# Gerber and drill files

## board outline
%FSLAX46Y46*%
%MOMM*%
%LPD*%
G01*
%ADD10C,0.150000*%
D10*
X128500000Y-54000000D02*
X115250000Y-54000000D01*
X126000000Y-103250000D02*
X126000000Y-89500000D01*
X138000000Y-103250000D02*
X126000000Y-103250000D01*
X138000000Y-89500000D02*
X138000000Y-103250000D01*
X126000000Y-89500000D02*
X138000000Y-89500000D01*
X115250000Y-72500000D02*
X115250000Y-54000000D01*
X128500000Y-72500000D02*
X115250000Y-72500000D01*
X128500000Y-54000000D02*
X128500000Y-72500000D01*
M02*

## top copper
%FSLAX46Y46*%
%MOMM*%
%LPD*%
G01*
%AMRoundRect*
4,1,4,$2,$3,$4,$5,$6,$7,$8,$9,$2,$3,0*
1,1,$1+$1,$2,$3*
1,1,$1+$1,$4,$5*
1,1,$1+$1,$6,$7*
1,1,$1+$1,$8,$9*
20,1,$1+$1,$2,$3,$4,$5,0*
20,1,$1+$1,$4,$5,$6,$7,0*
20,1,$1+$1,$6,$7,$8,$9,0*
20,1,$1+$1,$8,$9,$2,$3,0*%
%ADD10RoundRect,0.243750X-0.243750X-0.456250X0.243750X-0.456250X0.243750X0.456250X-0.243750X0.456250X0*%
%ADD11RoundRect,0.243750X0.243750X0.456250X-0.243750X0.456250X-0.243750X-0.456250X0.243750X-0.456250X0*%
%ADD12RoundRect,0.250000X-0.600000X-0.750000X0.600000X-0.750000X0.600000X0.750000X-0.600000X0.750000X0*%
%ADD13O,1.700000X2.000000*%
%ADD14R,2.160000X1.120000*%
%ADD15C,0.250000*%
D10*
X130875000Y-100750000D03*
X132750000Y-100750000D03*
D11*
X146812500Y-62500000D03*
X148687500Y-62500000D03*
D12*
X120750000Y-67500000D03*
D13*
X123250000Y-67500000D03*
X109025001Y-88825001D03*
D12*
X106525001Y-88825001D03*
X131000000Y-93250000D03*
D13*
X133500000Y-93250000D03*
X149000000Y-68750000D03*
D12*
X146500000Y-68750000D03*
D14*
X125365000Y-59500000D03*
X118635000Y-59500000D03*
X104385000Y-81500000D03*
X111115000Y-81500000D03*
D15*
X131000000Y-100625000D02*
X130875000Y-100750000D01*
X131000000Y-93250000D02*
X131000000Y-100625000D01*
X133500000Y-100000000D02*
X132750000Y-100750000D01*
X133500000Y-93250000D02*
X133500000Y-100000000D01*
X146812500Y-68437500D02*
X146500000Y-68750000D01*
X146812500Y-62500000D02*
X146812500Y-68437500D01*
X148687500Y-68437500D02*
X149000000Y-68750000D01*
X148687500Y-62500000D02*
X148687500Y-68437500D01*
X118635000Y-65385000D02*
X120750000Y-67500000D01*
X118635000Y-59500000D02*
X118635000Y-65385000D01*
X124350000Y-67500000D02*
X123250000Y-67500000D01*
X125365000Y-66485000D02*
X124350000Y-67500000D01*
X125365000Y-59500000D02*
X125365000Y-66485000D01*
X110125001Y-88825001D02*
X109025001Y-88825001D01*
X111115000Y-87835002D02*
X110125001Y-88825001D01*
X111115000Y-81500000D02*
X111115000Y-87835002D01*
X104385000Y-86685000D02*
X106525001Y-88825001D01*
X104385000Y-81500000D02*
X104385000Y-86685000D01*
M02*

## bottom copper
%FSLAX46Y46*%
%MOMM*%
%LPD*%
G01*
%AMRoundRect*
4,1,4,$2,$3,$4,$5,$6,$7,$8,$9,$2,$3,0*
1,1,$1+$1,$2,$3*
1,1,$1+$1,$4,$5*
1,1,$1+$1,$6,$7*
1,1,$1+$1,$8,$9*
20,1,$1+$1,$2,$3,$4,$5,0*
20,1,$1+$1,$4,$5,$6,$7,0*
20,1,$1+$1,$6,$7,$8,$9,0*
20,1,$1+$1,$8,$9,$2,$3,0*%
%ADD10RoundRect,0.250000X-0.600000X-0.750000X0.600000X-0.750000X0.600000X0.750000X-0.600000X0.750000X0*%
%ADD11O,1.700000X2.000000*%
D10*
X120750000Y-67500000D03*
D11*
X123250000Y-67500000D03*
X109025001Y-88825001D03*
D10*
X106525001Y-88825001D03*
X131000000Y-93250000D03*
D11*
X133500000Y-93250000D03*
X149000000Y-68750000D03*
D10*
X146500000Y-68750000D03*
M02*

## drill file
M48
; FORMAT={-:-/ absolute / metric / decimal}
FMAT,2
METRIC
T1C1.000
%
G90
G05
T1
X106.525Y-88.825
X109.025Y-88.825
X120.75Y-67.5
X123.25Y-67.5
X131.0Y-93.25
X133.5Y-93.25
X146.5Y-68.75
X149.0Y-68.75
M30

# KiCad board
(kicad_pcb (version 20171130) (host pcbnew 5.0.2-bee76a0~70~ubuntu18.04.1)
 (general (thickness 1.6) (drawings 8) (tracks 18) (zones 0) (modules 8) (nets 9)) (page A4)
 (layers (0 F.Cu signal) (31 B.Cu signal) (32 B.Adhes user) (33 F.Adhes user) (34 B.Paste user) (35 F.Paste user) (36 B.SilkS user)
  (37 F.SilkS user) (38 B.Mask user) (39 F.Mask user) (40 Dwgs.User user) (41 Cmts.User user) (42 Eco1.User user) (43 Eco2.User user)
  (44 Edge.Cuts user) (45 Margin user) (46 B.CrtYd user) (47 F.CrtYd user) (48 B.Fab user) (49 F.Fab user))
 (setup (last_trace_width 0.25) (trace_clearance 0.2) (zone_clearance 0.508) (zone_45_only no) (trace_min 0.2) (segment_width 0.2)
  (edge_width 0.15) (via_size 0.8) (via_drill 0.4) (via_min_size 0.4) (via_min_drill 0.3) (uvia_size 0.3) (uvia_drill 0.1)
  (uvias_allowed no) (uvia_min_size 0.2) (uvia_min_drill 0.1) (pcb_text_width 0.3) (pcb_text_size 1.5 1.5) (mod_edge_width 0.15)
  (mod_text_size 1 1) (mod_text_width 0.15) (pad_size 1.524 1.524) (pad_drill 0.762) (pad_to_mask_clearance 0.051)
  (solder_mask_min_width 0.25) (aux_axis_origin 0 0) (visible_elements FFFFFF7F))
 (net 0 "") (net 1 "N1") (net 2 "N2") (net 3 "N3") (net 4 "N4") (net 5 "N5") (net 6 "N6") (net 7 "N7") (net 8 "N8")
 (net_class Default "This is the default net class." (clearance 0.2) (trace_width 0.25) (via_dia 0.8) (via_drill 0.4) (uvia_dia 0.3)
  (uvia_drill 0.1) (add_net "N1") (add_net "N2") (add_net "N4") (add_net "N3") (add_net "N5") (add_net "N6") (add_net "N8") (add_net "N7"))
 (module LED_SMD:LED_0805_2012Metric (layer F.Cu) (at 131.8125 100.75)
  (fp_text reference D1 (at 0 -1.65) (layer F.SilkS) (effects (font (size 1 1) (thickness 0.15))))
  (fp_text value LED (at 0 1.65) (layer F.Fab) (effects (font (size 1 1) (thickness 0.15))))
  (pad 1 smd roundrect (at -0.9375 0) (size 0.975 1.4) (layers F.Cu F.Paste F.Mask) (roundrect_rratio 0.25) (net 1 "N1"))
  (pad 2 smd roundrect (at 0.9375 0) (size 0.975 1.4) (layers F.Cu F.Paste F.Mask) (roundrect_rratio 0.25) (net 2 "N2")))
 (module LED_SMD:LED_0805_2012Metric (layer F.Cu) (at 147.75 62.5 180)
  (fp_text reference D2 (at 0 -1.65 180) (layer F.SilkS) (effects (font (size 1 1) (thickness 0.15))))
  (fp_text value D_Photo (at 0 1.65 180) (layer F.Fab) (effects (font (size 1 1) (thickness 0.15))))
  (pad 2 smd roundrect (at 0.9375 0 180) (size 0.975 1.4) (layers F.Cu F.Paste F.Mask) (roundrect_rratio 0.25) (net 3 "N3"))
  (pad 1 smd roundrect (at -0.9375 0 180) (size 0.975 1.4) (layers F.Cu F.Paste F.Mask) (roundrect_rratio 0.25) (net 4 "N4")))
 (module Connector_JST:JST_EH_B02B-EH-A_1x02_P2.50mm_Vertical (layer F.Cu) (at 120.75 67.5)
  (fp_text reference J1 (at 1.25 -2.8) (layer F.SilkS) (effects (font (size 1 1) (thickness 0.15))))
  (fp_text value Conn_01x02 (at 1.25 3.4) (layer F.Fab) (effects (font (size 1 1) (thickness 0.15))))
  (pad 1 thru_hole roundrect (at 0 0) (size 1.7 2) (drill 1) (layers *.Cu *.Mask) (roundrect_rratio 0.147059) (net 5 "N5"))
  (pad 2 thru_hole oval (at 2.5 0) (size 1.7 2) (drill 1) (layers *.Cu *.Mask) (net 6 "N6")))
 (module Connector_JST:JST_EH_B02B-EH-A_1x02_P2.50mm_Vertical (layer F.Cu) (at 106.525001 88.825001)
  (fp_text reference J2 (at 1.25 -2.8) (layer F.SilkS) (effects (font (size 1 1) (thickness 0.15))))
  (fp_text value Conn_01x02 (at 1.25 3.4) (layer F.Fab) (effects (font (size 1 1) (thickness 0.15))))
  (pad 2 thru_hole oval (at 2.5 0) (size 1.7 2) (drill 1) (layers *.Cu *.Mask) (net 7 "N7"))
  (pad 1 thru_hole roundrect (at 0 0) (size 1.7 2) (drill 1) (layers *.Cu *.Mask) (roundrect_rratio 0.147059) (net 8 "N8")))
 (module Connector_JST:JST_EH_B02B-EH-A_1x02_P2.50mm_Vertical (layer F.Cu) (at 131 93.25)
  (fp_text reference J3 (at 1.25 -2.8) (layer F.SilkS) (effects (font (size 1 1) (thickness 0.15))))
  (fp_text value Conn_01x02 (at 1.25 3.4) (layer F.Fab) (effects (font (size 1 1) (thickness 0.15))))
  (pad 1 thru_hole roundrect (at 0 0) (size 1.7 2) (drill 1) (layers *.Cu *.Mask) (roundrect_rratio 0.147059) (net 1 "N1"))
  (pad 2 thru_hole oval (at 2.5 0) (size 1.7 2) (drill 1) (layers *.Cu *.Mask) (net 2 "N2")))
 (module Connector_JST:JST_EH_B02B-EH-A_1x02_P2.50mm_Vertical (layer F.Cu) (at 146.5 68.75)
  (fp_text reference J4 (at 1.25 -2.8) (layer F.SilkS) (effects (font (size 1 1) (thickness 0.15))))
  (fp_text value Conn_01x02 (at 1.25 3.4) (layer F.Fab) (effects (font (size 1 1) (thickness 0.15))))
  (pad 2 thru_hole oval (at 2.5 0) (size 1.7 2) (drill 1) (layers *.Cu *.Mask) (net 4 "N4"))
  (pad 1 thru_hole roundrect (at 0 0) (size 1.7 2) (drill 1) (layers *.Cu *.Mask) (roundrect_rratio 0.147059) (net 3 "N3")))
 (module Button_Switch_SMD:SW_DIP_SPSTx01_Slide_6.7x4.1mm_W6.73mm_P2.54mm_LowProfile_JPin (layer F.Cu) (at 122 59.5 180)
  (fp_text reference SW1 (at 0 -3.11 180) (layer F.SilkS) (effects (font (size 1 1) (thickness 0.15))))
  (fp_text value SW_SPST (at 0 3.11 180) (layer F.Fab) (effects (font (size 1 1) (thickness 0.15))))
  (pad 1 smd rect (at -3.365 0 180) (size 2.16 1.12) (layers F.Cu F.Paste F.Mask) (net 6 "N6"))
  (pad 2 smd rect (at 3.365 0 180) (size 2.16 1.12) (layers F.Cu F.Paste F.Mask) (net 5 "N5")))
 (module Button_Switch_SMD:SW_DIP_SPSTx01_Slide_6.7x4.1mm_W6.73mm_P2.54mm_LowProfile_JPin (layer F.Cu) (at 107.75 81.5 180)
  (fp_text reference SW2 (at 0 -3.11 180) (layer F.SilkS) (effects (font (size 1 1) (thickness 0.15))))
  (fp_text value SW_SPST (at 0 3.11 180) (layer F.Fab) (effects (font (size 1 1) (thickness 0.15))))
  (pad 2 smd rect (at 3.365 0 180) (size 2.16 1.12) (layers F.Cu F.Paste F.Mask) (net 8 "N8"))
  (pad 1 smd rect (at -3.365 0 180) (size 2.16 1.12) (layers F.Cu F.Paste F.Mask) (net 7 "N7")))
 (gr_line (start 128.5 54) (end 115.25 54) (layer Edge.Cuts) (width 0.15))
 (gr_line (start 126 103.25) (end 126 89.5) (layer Edge.Cuts) (width 0.15))
 (gr_line (start 138 103.25) (end 126 103.25) (layer Edge.Cuts) (width 0.15))
 (gr_line (start 138 89.5) (end 138 103.25) (layer Edge.Cuts) (width 0.15))
 (gr_line (start 126 89.5) (end 138 89.5) (layer Edge.Cuts) (width 0.15))
 (gr_line (start 115.25 72.5) (end 115.25 54) (layer Edge.Cuts) (width 0.15))
 (gr_line (start 128.5 72.5) (end 115.25 72.5) (layer Edge.Cuts) (width 0.15))
 (gr_line (start 128.5 54) (end 128.5 72.5) (layer Edge.Cuts) (width 0.15))
 (segment (start 131 100.625) (end 130.875 100.75) (width 0.25) (layer F.Cu) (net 1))
 (segment (start 131 93.25) (end 131 100.625) (width 0.25) (layer F.Cu) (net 1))
 (segment (start 133.5 100) (end 132.75 100.75) (width 0.25) (layer F.Cu) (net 2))
 (segment (start 133.5 93.25) (end 133.5 100) (width 0.25) (layer F.Cu) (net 2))
 (segment (start 146.8125 68.4375) (end 146.5 68.75) (width 0.25) (layer F.Cu) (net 3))
 (segment (start 146.8125 62.5) (end 146.8125 68.4375) (width 0.25) (layer F.Cu) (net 3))
 (segment (start 148.6875 68.4375) (end 149 68.75) (width 0.25) (layer F.Cu) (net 4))
 (segment (start 148.6875 62.5) (end 148.6875 68.4375) (width 0.25) (layer F.Cu) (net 4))
 (segment (start 118.635 65.385) (end 120.75 67.5) (width 0.25) (layer F.Cu) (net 5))
 (segment (start 118.635 59.5) (end 118.635 65.385) (width 0.25) (layer F.Cu) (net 5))
 (segment (start 124.35 67.5) (end 123.25 67.5) (width 0.25) (layer F.Cu) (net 6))
 (segment (start 125.365 66.485) (end 124.35 67.5) (width 0.25) (layer F.Cu) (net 6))
 (segment (start 125.365 59.5) (end 125.365 66.485) (width 0.25) (layer F.Cu) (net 6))
 (segment (start 110.125001 88.825001) (end 109.025001 88.825001) (width 0.25) (layer F.Cu) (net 7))
 (segment (start 111.115 87.835002) (end 110.125001 88.825001) (width 0.25) (layer F.Cu) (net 7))
 (segment (start 111.115 81.5) (end 111.115 87.835002) (width 0.25) (layer F.Cu) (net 7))
 (segment (start 104.385 86.685) (end 106.525001 88.825001) (width 0.25) (layer F.Cu) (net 8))
 (segment (start 104.385 81.5) (end 104.385 86.685) (width 0.25) (layer F.Cu) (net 8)))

